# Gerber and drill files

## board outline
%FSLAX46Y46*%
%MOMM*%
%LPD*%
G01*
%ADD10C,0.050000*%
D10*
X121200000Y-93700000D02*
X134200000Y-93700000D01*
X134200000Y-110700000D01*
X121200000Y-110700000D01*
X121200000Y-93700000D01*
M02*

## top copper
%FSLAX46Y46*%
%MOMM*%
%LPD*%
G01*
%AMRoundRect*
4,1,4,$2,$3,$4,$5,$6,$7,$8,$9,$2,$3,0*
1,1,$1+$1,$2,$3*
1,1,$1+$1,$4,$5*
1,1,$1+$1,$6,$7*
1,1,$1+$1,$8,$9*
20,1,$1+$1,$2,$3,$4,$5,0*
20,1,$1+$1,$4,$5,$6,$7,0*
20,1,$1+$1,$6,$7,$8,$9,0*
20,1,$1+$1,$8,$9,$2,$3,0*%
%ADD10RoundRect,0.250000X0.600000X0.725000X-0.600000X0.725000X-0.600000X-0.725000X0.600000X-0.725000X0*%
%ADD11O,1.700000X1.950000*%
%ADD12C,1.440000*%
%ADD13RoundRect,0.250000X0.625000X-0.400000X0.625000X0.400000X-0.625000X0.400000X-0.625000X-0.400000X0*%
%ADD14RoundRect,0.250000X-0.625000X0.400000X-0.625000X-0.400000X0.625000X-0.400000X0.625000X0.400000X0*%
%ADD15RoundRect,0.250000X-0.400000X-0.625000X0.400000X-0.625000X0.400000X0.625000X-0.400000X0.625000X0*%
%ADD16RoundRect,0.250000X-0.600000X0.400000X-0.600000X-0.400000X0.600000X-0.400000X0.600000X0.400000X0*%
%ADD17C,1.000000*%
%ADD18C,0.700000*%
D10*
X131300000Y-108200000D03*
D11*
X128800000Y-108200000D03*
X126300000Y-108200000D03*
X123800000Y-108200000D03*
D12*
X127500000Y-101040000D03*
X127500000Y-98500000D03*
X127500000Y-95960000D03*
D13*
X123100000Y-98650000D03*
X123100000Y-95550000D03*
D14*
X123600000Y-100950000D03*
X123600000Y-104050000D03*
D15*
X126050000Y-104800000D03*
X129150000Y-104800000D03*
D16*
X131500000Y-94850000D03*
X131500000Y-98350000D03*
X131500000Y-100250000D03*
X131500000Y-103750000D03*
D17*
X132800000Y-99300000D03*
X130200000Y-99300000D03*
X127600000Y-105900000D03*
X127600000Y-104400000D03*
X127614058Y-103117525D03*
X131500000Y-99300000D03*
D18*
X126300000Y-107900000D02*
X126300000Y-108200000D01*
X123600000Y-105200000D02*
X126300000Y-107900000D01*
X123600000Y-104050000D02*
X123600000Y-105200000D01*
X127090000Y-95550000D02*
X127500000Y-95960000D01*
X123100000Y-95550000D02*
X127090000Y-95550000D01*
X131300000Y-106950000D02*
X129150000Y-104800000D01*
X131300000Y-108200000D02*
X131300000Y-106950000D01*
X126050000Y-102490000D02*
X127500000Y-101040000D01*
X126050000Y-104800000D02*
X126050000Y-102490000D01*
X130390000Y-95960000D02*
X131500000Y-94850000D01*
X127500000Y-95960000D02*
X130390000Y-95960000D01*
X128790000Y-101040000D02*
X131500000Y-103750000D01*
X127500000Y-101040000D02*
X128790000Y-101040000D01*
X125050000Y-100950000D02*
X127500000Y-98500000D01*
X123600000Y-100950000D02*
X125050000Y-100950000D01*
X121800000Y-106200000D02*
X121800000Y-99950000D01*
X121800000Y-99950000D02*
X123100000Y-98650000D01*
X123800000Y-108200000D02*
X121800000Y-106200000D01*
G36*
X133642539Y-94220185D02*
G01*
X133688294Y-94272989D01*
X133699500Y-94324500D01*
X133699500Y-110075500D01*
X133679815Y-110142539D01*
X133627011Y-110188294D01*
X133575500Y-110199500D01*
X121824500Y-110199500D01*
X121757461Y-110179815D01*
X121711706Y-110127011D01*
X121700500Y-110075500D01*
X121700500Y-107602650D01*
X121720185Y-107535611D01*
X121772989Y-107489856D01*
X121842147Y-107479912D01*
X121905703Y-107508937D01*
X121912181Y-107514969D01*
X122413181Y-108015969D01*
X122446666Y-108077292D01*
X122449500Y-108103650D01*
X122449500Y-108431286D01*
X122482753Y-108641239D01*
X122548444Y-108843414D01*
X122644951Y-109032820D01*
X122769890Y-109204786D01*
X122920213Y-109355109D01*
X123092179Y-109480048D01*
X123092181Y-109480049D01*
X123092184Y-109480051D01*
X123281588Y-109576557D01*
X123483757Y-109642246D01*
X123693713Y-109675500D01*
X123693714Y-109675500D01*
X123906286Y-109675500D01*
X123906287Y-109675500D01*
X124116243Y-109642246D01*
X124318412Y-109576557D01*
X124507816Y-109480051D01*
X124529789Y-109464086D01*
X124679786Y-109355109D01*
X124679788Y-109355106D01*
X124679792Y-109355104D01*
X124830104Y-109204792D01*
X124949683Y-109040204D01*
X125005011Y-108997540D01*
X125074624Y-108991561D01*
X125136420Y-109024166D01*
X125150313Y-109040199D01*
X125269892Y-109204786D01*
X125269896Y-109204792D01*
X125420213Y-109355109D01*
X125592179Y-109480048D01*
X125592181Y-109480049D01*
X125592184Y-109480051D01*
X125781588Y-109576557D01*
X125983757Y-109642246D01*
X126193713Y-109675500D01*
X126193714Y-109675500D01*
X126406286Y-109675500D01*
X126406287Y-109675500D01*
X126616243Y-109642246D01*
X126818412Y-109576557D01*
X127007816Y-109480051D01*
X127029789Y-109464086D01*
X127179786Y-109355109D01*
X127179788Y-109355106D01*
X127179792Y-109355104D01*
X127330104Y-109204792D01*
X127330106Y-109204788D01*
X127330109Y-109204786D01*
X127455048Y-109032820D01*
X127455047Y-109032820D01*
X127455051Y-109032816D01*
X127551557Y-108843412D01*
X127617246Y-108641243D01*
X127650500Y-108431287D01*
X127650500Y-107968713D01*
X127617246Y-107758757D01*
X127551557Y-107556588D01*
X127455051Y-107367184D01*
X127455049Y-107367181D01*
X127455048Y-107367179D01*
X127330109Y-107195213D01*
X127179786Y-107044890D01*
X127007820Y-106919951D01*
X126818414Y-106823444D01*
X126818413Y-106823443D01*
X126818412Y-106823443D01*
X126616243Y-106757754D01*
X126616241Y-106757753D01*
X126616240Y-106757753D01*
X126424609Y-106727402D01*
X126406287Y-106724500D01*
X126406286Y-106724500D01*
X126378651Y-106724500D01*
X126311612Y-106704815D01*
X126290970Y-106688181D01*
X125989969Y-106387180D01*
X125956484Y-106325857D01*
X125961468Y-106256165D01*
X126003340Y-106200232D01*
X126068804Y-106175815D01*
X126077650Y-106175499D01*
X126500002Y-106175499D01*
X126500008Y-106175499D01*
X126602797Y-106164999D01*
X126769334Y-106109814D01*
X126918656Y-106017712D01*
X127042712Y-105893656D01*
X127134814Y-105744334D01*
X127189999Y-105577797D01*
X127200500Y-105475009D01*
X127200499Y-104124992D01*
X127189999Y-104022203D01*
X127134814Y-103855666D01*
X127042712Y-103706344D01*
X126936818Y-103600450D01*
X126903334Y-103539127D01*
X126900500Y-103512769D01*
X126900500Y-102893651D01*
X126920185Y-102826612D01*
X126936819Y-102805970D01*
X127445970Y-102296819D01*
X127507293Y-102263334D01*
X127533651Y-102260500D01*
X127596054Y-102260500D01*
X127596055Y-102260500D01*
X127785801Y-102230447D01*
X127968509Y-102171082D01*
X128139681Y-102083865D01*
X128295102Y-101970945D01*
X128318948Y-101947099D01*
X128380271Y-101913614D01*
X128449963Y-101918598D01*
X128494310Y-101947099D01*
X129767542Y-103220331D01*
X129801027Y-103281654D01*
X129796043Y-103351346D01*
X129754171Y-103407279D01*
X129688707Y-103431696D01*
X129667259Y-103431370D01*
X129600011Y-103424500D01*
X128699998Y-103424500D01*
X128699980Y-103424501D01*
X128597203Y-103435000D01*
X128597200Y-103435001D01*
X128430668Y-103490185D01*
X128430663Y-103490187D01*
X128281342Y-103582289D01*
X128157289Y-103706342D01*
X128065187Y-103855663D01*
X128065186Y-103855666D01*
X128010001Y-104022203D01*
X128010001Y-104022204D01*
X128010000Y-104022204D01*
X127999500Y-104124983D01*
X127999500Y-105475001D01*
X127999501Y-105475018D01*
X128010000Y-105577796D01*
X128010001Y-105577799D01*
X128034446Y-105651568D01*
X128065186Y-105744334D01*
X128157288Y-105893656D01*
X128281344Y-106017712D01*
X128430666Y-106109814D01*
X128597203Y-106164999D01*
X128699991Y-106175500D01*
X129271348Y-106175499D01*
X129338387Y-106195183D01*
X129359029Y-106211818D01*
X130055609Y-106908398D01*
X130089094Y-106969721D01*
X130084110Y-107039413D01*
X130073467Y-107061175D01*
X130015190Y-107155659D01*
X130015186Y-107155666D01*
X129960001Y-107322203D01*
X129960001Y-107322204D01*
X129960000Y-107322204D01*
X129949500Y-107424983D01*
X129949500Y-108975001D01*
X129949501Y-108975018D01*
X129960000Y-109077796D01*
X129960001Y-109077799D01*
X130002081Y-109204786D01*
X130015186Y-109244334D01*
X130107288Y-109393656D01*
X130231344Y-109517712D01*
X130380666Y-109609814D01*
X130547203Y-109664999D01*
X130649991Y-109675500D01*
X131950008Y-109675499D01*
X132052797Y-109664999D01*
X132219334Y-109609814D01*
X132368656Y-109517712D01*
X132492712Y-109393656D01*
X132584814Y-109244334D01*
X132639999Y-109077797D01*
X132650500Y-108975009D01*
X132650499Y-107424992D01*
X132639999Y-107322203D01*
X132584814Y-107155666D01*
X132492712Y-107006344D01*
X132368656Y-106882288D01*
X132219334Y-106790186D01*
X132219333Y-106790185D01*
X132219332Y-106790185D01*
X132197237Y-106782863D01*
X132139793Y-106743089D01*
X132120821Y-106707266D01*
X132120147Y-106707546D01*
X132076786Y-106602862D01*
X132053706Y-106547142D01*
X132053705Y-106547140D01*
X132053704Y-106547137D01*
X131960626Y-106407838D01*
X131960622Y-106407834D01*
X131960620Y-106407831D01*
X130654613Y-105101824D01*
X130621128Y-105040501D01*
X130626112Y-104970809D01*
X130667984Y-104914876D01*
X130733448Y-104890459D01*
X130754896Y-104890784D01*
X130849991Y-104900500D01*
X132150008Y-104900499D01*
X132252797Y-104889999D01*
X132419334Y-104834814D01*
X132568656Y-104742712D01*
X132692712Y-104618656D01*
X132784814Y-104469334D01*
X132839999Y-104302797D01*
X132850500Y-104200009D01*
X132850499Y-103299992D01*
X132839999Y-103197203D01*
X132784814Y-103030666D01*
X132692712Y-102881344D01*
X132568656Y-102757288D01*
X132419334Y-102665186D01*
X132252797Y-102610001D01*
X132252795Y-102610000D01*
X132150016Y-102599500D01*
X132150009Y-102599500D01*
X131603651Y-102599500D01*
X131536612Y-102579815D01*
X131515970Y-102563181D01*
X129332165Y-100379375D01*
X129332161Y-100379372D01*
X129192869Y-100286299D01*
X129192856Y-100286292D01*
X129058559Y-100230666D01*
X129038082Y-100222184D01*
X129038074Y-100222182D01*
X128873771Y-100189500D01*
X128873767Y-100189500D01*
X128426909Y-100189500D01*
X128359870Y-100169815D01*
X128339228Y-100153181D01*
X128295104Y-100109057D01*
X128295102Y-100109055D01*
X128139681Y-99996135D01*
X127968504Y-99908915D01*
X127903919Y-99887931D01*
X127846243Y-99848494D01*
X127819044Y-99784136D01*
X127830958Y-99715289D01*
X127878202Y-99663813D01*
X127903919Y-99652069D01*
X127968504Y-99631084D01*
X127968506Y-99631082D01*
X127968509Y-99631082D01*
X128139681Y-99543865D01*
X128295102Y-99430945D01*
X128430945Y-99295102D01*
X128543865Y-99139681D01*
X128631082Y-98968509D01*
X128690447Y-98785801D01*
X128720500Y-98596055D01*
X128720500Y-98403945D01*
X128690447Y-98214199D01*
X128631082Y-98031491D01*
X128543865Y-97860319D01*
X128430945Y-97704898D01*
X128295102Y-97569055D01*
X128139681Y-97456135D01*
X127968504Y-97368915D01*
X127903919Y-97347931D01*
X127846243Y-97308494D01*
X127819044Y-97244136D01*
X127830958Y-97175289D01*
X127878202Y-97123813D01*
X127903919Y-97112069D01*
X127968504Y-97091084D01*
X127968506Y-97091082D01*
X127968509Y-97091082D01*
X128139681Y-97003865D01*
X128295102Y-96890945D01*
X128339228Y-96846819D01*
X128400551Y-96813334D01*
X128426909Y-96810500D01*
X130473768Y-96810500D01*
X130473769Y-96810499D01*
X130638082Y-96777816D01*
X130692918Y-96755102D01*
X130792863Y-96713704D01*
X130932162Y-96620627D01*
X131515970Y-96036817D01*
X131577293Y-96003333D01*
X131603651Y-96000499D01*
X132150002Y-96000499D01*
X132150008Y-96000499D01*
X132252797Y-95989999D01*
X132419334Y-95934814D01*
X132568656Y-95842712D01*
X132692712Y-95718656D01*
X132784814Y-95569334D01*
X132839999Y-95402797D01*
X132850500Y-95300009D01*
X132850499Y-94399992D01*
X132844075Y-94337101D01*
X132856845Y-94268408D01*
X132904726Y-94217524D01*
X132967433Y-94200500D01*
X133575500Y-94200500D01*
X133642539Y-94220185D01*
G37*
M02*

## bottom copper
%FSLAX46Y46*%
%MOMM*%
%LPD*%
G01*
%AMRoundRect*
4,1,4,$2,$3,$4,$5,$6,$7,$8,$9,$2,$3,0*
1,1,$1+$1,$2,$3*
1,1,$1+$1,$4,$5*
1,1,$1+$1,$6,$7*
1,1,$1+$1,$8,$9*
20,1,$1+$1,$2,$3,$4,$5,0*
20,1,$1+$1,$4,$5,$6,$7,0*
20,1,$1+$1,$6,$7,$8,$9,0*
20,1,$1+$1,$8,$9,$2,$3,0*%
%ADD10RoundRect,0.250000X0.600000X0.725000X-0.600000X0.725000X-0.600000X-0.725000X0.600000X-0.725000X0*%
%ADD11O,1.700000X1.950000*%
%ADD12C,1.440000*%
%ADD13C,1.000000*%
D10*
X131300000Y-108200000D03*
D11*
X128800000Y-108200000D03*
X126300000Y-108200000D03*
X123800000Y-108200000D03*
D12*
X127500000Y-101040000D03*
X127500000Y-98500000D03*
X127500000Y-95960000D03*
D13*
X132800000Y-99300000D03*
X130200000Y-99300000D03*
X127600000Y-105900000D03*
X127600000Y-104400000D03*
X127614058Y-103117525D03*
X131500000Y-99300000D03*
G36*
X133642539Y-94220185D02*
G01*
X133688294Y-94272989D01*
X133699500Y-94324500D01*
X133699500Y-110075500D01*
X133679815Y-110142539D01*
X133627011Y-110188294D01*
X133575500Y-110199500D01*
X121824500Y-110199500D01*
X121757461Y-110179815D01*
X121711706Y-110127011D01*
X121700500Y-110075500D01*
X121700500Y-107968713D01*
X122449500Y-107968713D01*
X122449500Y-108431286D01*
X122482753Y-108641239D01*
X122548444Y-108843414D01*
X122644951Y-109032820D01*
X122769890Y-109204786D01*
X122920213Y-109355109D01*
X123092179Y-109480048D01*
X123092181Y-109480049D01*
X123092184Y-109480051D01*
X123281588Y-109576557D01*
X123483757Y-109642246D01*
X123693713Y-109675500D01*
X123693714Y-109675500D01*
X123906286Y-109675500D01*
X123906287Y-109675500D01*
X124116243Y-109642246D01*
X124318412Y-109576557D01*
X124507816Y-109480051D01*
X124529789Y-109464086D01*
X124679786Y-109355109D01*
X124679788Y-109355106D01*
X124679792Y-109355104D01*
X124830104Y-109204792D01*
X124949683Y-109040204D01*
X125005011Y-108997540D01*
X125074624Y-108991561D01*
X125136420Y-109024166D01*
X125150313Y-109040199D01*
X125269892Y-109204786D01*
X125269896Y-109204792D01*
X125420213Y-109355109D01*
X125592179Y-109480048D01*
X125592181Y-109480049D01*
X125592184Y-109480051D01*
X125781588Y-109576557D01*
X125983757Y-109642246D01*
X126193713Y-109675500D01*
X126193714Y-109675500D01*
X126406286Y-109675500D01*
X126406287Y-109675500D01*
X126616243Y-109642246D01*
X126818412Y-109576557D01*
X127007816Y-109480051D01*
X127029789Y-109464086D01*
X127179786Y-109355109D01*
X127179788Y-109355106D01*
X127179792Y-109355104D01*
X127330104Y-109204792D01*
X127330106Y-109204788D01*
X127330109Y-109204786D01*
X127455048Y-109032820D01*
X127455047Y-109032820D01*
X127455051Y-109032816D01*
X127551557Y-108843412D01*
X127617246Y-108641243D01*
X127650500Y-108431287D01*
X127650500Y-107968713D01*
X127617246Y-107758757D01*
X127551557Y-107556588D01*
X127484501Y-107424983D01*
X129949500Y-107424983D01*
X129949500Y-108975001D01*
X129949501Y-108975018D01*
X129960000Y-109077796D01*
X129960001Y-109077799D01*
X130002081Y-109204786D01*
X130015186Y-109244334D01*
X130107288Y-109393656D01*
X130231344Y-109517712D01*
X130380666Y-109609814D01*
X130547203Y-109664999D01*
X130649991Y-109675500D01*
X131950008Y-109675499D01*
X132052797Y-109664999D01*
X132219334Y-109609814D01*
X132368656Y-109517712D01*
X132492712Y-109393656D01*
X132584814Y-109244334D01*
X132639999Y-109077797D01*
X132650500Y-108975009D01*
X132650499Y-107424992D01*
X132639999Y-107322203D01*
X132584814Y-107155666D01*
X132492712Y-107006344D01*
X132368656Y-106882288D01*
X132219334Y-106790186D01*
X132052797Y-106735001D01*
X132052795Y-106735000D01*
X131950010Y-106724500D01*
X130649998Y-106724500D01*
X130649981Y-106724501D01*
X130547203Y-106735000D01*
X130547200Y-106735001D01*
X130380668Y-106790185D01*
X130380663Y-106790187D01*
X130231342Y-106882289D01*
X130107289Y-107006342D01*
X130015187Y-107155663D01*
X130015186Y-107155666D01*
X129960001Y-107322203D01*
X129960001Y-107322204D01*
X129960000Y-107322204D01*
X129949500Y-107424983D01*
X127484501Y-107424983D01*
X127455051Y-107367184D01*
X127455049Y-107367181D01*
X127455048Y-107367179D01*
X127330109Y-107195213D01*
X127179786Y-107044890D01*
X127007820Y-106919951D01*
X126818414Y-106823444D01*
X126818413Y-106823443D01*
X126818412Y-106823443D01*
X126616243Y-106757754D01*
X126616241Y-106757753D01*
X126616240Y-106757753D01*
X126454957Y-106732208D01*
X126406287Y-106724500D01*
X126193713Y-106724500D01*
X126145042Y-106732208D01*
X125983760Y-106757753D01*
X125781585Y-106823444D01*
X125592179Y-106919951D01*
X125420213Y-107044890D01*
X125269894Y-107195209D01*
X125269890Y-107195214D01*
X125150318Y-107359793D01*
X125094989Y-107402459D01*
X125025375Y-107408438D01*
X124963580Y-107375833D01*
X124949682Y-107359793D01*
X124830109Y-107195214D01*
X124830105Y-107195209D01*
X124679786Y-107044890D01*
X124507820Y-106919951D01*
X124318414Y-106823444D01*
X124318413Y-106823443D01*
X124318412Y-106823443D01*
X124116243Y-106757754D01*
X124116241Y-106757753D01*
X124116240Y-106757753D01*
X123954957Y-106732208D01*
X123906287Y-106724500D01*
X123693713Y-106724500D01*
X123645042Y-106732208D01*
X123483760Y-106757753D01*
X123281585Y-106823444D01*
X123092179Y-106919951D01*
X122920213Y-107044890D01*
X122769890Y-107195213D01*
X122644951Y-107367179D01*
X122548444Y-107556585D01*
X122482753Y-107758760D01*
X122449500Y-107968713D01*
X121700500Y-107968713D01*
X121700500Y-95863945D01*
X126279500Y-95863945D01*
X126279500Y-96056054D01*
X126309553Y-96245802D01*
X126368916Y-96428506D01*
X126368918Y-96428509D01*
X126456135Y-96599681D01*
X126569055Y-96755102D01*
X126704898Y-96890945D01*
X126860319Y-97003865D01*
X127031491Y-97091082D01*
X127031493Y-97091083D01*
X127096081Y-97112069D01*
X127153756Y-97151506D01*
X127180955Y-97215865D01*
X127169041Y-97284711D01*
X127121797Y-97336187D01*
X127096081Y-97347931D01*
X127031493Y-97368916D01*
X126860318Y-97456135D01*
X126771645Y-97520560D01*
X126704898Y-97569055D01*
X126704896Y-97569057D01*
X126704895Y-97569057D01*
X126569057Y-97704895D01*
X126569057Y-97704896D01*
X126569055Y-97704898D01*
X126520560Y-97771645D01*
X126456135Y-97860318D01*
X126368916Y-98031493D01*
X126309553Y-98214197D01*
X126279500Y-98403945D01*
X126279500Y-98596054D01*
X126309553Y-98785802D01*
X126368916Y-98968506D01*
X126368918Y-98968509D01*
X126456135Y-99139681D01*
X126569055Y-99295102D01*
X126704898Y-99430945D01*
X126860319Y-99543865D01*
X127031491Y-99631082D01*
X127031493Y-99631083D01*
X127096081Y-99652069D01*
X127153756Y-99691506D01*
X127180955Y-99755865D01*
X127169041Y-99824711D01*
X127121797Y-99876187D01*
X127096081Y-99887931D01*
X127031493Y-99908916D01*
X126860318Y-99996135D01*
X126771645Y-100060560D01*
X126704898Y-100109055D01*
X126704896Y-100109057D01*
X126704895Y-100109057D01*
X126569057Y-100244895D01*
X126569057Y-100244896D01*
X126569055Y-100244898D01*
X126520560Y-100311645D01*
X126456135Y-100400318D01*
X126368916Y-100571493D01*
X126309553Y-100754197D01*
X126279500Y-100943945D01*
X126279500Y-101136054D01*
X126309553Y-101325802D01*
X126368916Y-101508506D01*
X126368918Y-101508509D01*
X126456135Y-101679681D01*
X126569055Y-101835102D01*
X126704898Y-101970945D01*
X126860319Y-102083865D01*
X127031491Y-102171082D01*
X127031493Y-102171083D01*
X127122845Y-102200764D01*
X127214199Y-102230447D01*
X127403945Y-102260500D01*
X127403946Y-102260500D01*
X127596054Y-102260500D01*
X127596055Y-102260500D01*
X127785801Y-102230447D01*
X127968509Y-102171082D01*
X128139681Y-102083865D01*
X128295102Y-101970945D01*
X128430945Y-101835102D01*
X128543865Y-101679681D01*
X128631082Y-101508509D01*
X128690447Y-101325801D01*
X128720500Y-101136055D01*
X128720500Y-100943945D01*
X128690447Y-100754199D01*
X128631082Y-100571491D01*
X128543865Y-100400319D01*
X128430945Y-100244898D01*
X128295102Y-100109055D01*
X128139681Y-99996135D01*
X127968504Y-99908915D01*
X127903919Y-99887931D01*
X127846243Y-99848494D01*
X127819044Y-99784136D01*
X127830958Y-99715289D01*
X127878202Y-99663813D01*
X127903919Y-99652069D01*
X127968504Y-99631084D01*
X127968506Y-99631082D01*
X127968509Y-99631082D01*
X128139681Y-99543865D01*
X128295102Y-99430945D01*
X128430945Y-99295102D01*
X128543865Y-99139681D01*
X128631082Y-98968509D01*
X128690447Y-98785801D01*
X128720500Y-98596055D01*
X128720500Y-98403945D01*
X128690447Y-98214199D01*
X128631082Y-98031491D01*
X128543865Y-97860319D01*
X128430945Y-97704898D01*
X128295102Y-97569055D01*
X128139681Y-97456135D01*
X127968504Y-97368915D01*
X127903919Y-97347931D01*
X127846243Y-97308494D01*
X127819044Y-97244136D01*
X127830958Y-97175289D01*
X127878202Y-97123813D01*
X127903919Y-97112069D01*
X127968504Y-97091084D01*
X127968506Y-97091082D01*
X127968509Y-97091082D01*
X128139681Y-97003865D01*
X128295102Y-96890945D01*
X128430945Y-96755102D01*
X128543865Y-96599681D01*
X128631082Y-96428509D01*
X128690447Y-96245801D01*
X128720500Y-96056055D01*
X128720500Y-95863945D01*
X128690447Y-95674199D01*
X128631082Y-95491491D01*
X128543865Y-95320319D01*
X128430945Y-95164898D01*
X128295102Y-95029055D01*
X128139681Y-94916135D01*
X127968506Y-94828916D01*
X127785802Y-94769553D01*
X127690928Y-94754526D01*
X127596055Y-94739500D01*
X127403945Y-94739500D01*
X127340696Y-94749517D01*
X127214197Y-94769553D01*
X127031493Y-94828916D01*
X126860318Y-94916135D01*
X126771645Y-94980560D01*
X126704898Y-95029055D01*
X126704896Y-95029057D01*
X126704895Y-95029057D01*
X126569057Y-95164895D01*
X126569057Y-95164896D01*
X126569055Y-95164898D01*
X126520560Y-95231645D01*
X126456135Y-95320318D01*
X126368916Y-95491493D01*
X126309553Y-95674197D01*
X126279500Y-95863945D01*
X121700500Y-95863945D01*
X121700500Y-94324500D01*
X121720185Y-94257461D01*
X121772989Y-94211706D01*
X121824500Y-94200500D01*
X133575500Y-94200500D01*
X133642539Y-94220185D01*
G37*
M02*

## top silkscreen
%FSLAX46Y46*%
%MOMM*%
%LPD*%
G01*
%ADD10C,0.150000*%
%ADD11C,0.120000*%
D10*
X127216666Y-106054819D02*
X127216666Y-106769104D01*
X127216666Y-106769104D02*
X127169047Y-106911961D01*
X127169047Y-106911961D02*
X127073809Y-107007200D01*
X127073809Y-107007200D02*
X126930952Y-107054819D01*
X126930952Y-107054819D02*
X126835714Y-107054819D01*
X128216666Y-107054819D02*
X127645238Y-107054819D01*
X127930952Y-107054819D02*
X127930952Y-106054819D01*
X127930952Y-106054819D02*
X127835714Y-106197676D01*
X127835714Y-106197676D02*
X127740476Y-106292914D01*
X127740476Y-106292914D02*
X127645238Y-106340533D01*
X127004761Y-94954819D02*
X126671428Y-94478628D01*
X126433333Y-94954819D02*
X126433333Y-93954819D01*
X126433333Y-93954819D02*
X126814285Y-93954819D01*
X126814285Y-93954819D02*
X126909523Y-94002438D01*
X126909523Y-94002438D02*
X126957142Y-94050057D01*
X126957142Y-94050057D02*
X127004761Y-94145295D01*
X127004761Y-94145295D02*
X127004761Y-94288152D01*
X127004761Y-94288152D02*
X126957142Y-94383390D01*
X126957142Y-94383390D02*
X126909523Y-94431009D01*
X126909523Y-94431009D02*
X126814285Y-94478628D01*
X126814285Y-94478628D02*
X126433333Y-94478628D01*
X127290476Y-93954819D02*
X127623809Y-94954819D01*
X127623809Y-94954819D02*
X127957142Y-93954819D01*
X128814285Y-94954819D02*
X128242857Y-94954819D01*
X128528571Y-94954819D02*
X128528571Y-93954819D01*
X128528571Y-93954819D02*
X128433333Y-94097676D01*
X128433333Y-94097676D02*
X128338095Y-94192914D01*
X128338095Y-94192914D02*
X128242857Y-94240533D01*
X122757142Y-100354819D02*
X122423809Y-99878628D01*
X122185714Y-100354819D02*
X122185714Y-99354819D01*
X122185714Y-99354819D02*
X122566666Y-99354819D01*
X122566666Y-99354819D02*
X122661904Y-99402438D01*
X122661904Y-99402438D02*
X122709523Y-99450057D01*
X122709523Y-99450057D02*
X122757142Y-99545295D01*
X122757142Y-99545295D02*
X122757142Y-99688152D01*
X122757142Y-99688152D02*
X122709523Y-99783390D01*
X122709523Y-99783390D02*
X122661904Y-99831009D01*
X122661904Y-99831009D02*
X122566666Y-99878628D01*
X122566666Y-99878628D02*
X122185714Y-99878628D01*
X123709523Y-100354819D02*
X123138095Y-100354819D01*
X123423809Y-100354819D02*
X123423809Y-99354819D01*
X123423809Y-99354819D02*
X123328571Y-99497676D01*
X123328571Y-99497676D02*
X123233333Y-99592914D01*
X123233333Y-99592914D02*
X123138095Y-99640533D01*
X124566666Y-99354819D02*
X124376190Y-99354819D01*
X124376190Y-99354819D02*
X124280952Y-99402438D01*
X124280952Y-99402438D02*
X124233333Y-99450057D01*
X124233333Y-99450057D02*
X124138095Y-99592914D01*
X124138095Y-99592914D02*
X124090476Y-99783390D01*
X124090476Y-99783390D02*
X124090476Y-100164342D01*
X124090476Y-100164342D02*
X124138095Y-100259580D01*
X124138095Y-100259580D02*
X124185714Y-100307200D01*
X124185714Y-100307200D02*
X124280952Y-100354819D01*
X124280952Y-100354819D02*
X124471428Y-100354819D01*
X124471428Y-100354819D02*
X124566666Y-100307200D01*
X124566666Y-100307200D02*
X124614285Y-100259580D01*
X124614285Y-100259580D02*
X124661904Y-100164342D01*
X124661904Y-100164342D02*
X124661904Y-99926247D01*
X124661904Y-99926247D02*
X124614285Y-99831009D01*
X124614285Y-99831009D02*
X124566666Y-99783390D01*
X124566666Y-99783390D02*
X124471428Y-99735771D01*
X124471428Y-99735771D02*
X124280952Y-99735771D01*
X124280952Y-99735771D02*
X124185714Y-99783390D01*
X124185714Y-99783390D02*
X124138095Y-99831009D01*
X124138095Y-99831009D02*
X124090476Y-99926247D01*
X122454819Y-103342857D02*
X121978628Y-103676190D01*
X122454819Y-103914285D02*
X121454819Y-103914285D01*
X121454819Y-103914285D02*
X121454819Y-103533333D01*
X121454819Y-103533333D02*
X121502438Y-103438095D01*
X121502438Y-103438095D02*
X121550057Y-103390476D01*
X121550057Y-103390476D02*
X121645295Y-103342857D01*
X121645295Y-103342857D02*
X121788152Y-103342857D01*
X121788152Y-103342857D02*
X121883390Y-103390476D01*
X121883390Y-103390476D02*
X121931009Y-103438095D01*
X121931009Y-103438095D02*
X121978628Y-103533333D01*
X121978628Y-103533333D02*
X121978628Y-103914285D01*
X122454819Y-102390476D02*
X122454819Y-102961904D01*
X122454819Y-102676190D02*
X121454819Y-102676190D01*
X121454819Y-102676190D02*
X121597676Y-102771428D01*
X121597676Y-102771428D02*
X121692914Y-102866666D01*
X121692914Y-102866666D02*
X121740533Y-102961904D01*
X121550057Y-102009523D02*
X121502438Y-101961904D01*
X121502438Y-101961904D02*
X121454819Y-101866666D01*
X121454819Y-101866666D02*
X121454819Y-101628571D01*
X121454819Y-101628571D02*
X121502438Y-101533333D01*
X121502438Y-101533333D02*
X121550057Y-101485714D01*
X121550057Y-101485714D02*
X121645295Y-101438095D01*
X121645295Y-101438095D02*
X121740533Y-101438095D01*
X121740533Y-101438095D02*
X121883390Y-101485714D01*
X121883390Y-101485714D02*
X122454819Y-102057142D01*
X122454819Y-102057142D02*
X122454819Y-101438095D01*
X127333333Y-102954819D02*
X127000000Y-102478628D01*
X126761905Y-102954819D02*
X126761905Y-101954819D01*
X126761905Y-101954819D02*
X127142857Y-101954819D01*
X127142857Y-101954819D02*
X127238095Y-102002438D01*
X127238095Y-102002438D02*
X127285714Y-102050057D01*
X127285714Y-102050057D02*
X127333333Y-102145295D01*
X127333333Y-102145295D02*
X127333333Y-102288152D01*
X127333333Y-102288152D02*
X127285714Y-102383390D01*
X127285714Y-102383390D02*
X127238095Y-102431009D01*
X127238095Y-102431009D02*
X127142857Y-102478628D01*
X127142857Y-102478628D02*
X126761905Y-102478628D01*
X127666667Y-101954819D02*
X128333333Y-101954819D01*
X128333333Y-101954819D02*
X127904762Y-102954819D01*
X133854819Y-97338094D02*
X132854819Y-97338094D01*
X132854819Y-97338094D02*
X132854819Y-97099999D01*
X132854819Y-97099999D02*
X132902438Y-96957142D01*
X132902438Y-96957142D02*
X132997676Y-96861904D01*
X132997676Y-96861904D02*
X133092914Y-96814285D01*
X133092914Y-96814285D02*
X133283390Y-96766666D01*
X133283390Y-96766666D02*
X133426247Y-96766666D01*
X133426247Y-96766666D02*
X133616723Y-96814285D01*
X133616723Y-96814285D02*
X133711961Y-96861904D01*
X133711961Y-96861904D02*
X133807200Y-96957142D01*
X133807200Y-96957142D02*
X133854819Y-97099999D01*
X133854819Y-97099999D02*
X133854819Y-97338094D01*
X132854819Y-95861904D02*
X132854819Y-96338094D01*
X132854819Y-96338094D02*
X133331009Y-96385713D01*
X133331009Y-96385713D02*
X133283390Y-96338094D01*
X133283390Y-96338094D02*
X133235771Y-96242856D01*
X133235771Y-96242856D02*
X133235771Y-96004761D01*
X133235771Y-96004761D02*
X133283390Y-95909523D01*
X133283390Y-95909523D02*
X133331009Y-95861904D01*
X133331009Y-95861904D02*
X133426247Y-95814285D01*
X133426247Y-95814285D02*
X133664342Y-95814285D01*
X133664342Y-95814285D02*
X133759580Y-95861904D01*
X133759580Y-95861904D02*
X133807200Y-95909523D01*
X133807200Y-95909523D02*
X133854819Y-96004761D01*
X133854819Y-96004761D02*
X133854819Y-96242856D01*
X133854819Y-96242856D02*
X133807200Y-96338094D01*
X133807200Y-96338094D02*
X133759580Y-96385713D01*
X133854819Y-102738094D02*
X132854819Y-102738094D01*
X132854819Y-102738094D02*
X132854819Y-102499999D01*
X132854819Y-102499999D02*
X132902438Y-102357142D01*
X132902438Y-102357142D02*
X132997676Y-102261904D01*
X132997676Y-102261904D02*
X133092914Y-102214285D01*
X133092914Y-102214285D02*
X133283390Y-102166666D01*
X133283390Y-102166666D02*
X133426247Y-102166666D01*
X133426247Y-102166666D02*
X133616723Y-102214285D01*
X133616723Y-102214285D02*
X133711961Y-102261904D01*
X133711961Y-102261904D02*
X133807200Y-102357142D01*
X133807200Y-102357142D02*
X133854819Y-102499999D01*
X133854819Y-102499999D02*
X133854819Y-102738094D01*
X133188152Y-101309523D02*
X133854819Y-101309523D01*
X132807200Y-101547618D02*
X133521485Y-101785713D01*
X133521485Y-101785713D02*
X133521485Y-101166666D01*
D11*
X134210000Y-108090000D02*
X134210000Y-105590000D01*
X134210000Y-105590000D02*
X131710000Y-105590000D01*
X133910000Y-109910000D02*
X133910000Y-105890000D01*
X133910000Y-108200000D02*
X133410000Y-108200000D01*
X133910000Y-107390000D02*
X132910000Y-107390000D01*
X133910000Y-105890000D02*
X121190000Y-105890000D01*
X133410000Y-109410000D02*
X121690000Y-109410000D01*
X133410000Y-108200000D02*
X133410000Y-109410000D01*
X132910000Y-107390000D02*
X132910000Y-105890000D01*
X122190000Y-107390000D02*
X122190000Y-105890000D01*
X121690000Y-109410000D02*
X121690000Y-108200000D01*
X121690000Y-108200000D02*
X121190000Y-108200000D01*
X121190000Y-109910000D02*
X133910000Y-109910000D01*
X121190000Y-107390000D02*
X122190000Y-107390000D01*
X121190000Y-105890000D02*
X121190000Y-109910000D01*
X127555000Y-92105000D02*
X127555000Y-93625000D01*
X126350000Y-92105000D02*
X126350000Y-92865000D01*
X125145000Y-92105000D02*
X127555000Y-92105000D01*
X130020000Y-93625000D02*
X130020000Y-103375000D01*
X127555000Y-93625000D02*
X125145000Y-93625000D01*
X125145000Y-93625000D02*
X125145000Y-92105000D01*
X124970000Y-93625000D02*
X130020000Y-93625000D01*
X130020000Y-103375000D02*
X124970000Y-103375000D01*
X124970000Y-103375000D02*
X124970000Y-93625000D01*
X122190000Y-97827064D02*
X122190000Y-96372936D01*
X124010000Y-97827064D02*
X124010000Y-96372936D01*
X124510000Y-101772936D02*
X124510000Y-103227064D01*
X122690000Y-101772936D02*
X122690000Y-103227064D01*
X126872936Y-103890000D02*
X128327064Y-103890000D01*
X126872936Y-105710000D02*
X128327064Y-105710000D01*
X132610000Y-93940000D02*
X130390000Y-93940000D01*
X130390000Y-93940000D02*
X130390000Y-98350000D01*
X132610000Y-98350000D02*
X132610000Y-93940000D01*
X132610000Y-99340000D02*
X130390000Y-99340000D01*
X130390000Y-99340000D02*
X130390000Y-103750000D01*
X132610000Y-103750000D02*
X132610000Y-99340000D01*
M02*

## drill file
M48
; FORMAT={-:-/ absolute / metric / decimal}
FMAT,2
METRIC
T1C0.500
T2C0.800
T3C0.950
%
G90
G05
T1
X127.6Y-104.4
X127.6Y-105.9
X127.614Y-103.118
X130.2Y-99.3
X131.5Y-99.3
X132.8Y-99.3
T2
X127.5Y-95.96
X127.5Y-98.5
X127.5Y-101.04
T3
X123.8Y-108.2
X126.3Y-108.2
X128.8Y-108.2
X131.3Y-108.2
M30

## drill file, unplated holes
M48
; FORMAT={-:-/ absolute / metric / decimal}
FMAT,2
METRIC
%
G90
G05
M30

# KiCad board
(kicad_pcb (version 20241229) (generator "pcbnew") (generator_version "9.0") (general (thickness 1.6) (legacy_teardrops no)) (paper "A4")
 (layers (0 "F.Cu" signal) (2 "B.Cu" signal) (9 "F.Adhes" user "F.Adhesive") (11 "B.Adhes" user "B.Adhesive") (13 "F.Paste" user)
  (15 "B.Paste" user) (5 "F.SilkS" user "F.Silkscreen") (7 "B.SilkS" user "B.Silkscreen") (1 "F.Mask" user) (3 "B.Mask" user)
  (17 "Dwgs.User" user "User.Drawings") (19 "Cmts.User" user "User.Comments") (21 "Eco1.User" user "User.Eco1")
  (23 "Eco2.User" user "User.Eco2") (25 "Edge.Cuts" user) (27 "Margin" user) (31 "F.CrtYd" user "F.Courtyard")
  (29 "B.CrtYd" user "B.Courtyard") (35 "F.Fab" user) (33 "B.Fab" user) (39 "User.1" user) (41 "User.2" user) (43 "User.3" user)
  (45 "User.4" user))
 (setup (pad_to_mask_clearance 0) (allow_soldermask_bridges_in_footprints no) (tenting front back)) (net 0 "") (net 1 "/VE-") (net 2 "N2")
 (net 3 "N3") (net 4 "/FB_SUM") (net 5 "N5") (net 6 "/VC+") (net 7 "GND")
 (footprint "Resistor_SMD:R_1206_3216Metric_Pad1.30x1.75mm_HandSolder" (layer "F.Cu") (at 123.1 97.1 90)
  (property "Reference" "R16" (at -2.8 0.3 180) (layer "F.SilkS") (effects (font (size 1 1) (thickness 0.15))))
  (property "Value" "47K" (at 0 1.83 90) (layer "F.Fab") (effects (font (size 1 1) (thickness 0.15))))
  (fp_line (start -0.727064 -0.91) (end 0.727064 -0.91) (stroke (width 0.12) (type solid)) (layer "F.SilkS"))
  (fp_line (start -0.727064 0.91) (end 0.727064 0.91) (stroke (width 0.12) (type solid)) (layer "F.SilkS"))
  (pad "1" smd roundrect (at -1.55 0 90) (size 1.3 1.75) (layers "F.Cu" "F.Mask" "F.Paste") (roundrect_rratio 0.192308) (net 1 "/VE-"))
  (pad "2" smd roundrect (at 1.55 0 90) (size 1.3 1.75) (layers "F.Cu" "F.Mask" "F.Paste") (roundrect_rratio 0.192308) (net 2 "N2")))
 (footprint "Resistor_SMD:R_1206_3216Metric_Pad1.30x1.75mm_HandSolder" (layer "F.Cu") (at 123.6 102.5 -90)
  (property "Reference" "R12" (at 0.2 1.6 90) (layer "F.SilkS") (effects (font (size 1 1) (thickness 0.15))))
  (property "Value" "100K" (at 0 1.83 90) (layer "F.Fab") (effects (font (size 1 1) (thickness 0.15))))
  (fp_line (start -0.727064 0.91) (end 0.727064 0.91) (stroke (width 0.12) (type solid)) (layer "F.SilkS"))
  (fp_line (start -0.727064 -0.91) (end 0.727064 -0.91) (stroke (width 0.12) (type solid)) (layer "F.SilkS"))
  (pad "1" smd roundrect (at -1.55 0 270) (size 1.3 1.75) (layers "F.Cu" "F.Mask" "F.Paste") (roundrect_rratio 0.192308) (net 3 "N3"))
  (pad "2" smd roundrect (at 1.55 0 270) (size 1.3 1.75) (layers "F.Cu" "F.Mask" "F.Paste") (roundrect_rratio 0.192308) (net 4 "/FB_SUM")))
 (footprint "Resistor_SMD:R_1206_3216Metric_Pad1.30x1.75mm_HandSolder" (layer "F.Cu") (at 127.6 104.8)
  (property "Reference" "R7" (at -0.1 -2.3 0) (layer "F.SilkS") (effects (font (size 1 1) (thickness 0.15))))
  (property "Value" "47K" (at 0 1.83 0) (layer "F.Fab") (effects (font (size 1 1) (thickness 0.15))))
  (fp_line (start -0.727064 -0.91) (end 0.727064 -0.91) (stroke (width 0.12) (type solid)) (layer "F.SilkS"))
  (fp_line (start -0.727064 0.91) (end 0.727064 0.91) (stroke (width 0.12) (type solid)) (layer "F.SilkS"))
  (pad "1" smd roundrect (at -1.55 0) (size 1.3 1.75) (layers "F.Cu" "F.Mask" "F.Paste") (roundrect_rratio 0.192308) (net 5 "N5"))
  (pad "2" smd roundrect (at 1.55 0) (size 1.3 1.75) (layers "F.Cu" "F.Mask" "F.Paste") (roundrect_rratio 0.192308) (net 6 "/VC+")))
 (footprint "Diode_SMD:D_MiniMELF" (layer "F.Cu") (at 131.5 102 -90)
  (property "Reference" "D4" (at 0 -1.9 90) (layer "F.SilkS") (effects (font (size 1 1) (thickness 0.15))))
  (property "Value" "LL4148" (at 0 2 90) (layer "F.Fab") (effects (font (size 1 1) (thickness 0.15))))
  (fp_line (start -2.66 1.11) (end 1.75 1.11) (stroke (width 0.12) (type solid)) (layer "F.SilkS"))
  (fp_line (start -2.66 -1.11) (end -2.66 1.11) (stroke (width 0.12) (type solid)) (layer "F.SilkS"))
  (fp_line (start 1.75 -1.11) (end -2.66 -1.11) (stroke (width 0.12) (type solid)) (layer "F.SilkS"))
  (pad "1" smd roundrect (at -1.75 0 270) (size 1.3 1.7) (layers "F.Cu" "F.Mask" "F.Paste") (roundrect_rratio 0.1923076923) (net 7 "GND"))
  (pad "2" smd roundrect (at 1.75 0 270) (size 1.3 1.7) (layers "F.Cu" "F.Mask" "F.Paste") (roundrect_rratio 0.1923076923) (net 5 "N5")))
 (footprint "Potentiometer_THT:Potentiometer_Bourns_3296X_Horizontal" (layer "F.Cu") (at 127.5 101.04 -90)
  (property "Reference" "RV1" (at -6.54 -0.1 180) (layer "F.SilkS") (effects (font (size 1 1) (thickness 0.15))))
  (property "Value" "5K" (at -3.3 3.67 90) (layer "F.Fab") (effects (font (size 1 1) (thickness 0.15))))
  (fp_line (start -7.415 2.53) (end -7.415 -2.52) (stroke (width 0.12) (type solid)) (layer "F.SilkS"))
  (fp_line (start 2.335 2.53) (end -7.415 2.53) (stroke (width 0.12) (type solid)) (layer "F.SilkS"))
  (fp_line (start -8.935 2.355) (end -8.935 -0.055) (stroke (width 0.12) (type solid)) (layer "F.SilkS"))
  (fp_line (start -7.415 2.355) (end -8.935 2.355) (stroke (width 0.12) (type solid)) (layer "F.SilkS"))
  (fp_line (start -8.935 1.15) (end -8.175 1.15) (stroke (width 0.12) (type solid)) (layer "F.SilkS"))
  (fp_line (start -8.935 -0.055) (end -7.415 -0.055) (stroke (width 0.12) (type solid)) (layer "F.SilkS"))
  (fp_line (start -7.415 -0.055) (end -7.415 2.355) (stroke (width 0.12) (type solid)) (layer "F.SilkS"))
  (fp_line (start -7.415 -2.52) (end 2.335 -2.52) (stroke (width 0.12) (type solid)) (layer "F.SilkS"))
  (fp_line (start 2.335 -2.52) (end 2.335 2.53) (stroke (width 0.12) (type solid)) (layer "F.SilkS"))
  (pad "1" thru_hole circle (at 0 0 270) (size 1.44 1.44) (drill 0.8) (layers "*.Cu" "*.Mask") (remove_unused_layers no) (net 5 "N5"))
  (pad "2" thru_hole circle (at -2.54 0 270) (size 1.44 1.44) (drill 0.8) (layers "*.Cu" "*.Mask") (remove_unused_layers no) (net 3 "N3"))
  (pad "3" thru_hole circle (at -5.08 0 270) (size 1.44 1.44) (drill 0.8) (layers "*.Cu" "*.Mask") (remove_unused_layers no) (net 2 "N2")))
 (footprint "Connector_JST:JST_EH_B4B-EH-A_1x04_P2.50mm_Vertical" (layer "F.Cu") (at 131.3 108.2 180)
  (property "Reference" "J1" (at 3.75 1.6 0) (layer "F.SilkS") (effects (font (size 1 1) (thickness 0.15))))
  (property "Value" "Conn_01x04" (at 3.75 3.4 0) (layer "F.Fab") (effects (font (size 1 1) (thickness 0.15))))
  (fp_line (start 10.11 2.31) (end 10.11 -1.71) (stroke (width 0.12) (type solid)) (layer "F.SilkS"))
  (fp_line (start 10.11 0.81) (end 9.11 0.81) (stroke (width 0.12) (type solid)) (layer "F.SilkS"))
  (fp_line (start 10.11 -1.71) (end -2.61 -1.71) (stroke (width 0.12) (type solid)) (layer "F.SilkS"))
  (fp_line (start 9.61 0) (end 10.11 0) (stroke (width 0.12) (type solid)) (layer "F.SilkS"))
  (fp_line (start 9.61 -1.21) (end 9.61 0) (stroke (width 0.12) (type solid)) (layer "F.SilkS"))
  (fp_line (start 9.11 0.81) (end 9.11 2.31) (stroke (width 0.12) (type solid)) (layer "F.SilkS"))
  (fp_line (start -1.61 0.81) (end -1.61 2.31) (stroke (width 0.12) (type solid)) (layer "F.SilkS"))
  (fp_line (start -2.11 0) (end -2.11 -1.21) (stroke (width 0.12) (type solid)) (layer "F.SilkS"))
  (fp_line (start -2.11 -1.21) (end 9.61 -1.21) (stroke (width 0.12) (type solid)) (layer "F.SilkS"))
  (fp_line (start -2.61 2.31) (end 10.11 2.31) (stroke (width 0.12) (type solid)) (layer "F.SilkS"))
  (fp_line (start -2.61 0.81) (end -1.61 0.81) (stroke (width 0.12) (type solid)) (layer "F.SilkS"))
  (fp_line (start -2.61 0) (end -2.11 0) (stroke (width 0.12) (type solid)) (layer "F.SilkS"))
  (fp_line (start -2.61 -1.71) (end -2.61 2.31) (stroke (width 0.12) (type solid)) (layer "F.SilkS"))
  (fp_line (start -2.91 2.61) (end -0.41 2.61) (stroke (width 0.12) (type solid)) (layer "F.SilkS"))
  (fp_line (start -2.91 0.11) (end -2.91 2.61) (stroke (width 0.12) (type solid)) (layer "F.SilkS"))
  (pad "1" thru_hole roundrect (at 0 0 180) (size 1.7 1.95) (drill 0.95) (layers "*.Cu" "*.Mask") (remove_unused_layers no)
   (roundrect_rratio 0.147059) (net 6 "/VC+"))
  (pad "2" thru_hole oval (at 2.5 0 180) (size 1.7 1.95) (drill 0.95) (layers "*.Cu" "*.Mask") (remove_unused_layers no) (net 7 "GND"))
  (pad "3" thru_hole oval (at 5 0 180) (size 1.7 1.95) (drill 0.95) (layers "*.Cu" "*.Mask") (remove_unused_layers no) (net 4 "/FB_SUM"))
  (pad "4" thru_hole oval (at 7.5 0 180) (size 1.7 1.95) (drill 0.95) (layers "*.Cu" "*.Mask") (remove_unused_layers no) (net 1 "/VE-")))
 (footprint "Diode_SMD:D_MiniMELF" (layer "F.Cu") (at 131.5 96.6 -90)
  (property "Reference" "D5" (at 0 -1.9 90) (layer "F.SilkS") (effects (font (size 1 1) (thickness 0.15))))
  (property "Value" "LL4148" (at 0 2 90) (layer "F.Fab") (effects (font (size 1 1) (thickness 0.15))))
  (fp_line (start -2.66 1.11) (end 1.75 1.11) (stroke (width 0.12) (type solid)) (layer "F.SilkS"))
  (fp_line (start -2.66 -1.11) (end -2.66 1.11) (stroke (width 0.12) (type solid)) (layer "F.SilkS"))
  (fp_line (start 1.75 -1.11) (end -2.66 -1.11) (stroke (width 0.12) (type solid)) (layer "F.SilkS"))
  (pad "1" smd roundrect (at -1.75 0 270) (size 1.3 1.7) (layers "F.Cu" "F.Mask" "F.Paste") (roundrect_rratio 0.1923076923) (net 2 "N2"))
  (pad "2" smd roundrect (at 1.75 0 270) (size 1.3 1.7) (layers "F.Cu" "F.Mask" "F.Paste") (roundrect_rratio 0.1923076923) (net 7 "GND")))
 (gr_rect (start 121.2 93.7) (end 134.2 110.7) (stroke (width 0.05) (type solid)) (fill no) (layer "Edge.Cuts"))
 (segment (start 126.05 102.49) (end 127.5 101.04) (width 0.7) (layer "F.Cu") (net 5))
 (segment (start 127.5 101.04) (end 128.79 101.04) (width 0.7) (layer "F.Cu") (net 5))
 (segment (start 128.79 101.04) (end 131.5 103.75) (width 0.7) (layer "F.Cu") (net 5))
 (segment (start 126.05 104.8) (end 126.05 102.49) (width 0.7) (layer "F.Cu") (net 5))
 (via (at 131.5 99.3) (size 1) (drill 0.5) (layers "F.Cu" "B.Cu") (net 7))
 (via (at 127.614058 103.117525) (size 1) (drill 0.5) (layers "F.Cu" "B.Cu") (free yes) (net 7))
 (via (at 132.8 99.3) (size 1) (drill 0.5) (layers "F.Cu" "B.Cu") (free yes) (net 7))
 (via (at 130.2 99.3) (size 1) (drill 0.5) (layers "F.Cu" "B.Cu") (free yes) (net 7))
 (via (at 127.6 104.4) (size 1) (drill 0.5) (layers "F.Cu" "B.Cu") (free yes) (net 7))
 (via (at 127.6 105.9) (size 1) (drill 0.5) (layers "F.Cu" "B.Cu") (free yes) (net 7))
 (segment (start 127.09 95.55) (end 127.5 95.96) (width 0.7) (layer "F.Cu") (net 2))
 (segment (start 130.39 95.96) (end 131.5 94.85) (width 0.7) (layer "F.Cu") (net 2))
 (segment (start 123.1 95.55) (end 127.09 95.55) (width 0.7) (layer "F.Cu") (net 2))
 (segment (start 127.5 95.96) (end 130.39 95.96) (width 0.7) (layer "F.Cu") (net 2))
 (segment (start 131.3 108.2) (end 131.3 106.95) (width 0.7) (layer "F.Cu") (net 6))
 (segment (start 131.3 106.95) (end 129.15 104.8) (width 0.7) (layer "F.Cu") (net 6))
 (segment (start 125.05 100.95) (end 127.5 98.5) (width 0.7) (layer "F.Cu") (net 3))
 (segment (start 123.6 100.95) (end 125.05 100.95) (width 0.7) (layer "F.Cu") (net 3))
 (segment (start 126.3 107.9) (end 126.3 108.2) (width 0.7) (layer "F.Cu") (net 4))
 (segment (start 123.6 104.05) (end 123.6 105.2) (width 0.7) (layer "F.Cu") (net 4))
 (segment (start 123.6 105.2) (end 126.3 107.9) (width 0.7) (layer "F.Cu") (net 4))
 (segment (start 121.8 99.95) (end 123.1 98.65) (width 0.7) (layer "F.Cu") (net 1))
 (segment (start 123.8 108.2) (end 121.8 106.2) (width 0.7) (layer "F.Cu") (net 1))
 (segment (start 121.8 106.2) (end 121.8 99.95) (width 0.7) (layer "F.Cu") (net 1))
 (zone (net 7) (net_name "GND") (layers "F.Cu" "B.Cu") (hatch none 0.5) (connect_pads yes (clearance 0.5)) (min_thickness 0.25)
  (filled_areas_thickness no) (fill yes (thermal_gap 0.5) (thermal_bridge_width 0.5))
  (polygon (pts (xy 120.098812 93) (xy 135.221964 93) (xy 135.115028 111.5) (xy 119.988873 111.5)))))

